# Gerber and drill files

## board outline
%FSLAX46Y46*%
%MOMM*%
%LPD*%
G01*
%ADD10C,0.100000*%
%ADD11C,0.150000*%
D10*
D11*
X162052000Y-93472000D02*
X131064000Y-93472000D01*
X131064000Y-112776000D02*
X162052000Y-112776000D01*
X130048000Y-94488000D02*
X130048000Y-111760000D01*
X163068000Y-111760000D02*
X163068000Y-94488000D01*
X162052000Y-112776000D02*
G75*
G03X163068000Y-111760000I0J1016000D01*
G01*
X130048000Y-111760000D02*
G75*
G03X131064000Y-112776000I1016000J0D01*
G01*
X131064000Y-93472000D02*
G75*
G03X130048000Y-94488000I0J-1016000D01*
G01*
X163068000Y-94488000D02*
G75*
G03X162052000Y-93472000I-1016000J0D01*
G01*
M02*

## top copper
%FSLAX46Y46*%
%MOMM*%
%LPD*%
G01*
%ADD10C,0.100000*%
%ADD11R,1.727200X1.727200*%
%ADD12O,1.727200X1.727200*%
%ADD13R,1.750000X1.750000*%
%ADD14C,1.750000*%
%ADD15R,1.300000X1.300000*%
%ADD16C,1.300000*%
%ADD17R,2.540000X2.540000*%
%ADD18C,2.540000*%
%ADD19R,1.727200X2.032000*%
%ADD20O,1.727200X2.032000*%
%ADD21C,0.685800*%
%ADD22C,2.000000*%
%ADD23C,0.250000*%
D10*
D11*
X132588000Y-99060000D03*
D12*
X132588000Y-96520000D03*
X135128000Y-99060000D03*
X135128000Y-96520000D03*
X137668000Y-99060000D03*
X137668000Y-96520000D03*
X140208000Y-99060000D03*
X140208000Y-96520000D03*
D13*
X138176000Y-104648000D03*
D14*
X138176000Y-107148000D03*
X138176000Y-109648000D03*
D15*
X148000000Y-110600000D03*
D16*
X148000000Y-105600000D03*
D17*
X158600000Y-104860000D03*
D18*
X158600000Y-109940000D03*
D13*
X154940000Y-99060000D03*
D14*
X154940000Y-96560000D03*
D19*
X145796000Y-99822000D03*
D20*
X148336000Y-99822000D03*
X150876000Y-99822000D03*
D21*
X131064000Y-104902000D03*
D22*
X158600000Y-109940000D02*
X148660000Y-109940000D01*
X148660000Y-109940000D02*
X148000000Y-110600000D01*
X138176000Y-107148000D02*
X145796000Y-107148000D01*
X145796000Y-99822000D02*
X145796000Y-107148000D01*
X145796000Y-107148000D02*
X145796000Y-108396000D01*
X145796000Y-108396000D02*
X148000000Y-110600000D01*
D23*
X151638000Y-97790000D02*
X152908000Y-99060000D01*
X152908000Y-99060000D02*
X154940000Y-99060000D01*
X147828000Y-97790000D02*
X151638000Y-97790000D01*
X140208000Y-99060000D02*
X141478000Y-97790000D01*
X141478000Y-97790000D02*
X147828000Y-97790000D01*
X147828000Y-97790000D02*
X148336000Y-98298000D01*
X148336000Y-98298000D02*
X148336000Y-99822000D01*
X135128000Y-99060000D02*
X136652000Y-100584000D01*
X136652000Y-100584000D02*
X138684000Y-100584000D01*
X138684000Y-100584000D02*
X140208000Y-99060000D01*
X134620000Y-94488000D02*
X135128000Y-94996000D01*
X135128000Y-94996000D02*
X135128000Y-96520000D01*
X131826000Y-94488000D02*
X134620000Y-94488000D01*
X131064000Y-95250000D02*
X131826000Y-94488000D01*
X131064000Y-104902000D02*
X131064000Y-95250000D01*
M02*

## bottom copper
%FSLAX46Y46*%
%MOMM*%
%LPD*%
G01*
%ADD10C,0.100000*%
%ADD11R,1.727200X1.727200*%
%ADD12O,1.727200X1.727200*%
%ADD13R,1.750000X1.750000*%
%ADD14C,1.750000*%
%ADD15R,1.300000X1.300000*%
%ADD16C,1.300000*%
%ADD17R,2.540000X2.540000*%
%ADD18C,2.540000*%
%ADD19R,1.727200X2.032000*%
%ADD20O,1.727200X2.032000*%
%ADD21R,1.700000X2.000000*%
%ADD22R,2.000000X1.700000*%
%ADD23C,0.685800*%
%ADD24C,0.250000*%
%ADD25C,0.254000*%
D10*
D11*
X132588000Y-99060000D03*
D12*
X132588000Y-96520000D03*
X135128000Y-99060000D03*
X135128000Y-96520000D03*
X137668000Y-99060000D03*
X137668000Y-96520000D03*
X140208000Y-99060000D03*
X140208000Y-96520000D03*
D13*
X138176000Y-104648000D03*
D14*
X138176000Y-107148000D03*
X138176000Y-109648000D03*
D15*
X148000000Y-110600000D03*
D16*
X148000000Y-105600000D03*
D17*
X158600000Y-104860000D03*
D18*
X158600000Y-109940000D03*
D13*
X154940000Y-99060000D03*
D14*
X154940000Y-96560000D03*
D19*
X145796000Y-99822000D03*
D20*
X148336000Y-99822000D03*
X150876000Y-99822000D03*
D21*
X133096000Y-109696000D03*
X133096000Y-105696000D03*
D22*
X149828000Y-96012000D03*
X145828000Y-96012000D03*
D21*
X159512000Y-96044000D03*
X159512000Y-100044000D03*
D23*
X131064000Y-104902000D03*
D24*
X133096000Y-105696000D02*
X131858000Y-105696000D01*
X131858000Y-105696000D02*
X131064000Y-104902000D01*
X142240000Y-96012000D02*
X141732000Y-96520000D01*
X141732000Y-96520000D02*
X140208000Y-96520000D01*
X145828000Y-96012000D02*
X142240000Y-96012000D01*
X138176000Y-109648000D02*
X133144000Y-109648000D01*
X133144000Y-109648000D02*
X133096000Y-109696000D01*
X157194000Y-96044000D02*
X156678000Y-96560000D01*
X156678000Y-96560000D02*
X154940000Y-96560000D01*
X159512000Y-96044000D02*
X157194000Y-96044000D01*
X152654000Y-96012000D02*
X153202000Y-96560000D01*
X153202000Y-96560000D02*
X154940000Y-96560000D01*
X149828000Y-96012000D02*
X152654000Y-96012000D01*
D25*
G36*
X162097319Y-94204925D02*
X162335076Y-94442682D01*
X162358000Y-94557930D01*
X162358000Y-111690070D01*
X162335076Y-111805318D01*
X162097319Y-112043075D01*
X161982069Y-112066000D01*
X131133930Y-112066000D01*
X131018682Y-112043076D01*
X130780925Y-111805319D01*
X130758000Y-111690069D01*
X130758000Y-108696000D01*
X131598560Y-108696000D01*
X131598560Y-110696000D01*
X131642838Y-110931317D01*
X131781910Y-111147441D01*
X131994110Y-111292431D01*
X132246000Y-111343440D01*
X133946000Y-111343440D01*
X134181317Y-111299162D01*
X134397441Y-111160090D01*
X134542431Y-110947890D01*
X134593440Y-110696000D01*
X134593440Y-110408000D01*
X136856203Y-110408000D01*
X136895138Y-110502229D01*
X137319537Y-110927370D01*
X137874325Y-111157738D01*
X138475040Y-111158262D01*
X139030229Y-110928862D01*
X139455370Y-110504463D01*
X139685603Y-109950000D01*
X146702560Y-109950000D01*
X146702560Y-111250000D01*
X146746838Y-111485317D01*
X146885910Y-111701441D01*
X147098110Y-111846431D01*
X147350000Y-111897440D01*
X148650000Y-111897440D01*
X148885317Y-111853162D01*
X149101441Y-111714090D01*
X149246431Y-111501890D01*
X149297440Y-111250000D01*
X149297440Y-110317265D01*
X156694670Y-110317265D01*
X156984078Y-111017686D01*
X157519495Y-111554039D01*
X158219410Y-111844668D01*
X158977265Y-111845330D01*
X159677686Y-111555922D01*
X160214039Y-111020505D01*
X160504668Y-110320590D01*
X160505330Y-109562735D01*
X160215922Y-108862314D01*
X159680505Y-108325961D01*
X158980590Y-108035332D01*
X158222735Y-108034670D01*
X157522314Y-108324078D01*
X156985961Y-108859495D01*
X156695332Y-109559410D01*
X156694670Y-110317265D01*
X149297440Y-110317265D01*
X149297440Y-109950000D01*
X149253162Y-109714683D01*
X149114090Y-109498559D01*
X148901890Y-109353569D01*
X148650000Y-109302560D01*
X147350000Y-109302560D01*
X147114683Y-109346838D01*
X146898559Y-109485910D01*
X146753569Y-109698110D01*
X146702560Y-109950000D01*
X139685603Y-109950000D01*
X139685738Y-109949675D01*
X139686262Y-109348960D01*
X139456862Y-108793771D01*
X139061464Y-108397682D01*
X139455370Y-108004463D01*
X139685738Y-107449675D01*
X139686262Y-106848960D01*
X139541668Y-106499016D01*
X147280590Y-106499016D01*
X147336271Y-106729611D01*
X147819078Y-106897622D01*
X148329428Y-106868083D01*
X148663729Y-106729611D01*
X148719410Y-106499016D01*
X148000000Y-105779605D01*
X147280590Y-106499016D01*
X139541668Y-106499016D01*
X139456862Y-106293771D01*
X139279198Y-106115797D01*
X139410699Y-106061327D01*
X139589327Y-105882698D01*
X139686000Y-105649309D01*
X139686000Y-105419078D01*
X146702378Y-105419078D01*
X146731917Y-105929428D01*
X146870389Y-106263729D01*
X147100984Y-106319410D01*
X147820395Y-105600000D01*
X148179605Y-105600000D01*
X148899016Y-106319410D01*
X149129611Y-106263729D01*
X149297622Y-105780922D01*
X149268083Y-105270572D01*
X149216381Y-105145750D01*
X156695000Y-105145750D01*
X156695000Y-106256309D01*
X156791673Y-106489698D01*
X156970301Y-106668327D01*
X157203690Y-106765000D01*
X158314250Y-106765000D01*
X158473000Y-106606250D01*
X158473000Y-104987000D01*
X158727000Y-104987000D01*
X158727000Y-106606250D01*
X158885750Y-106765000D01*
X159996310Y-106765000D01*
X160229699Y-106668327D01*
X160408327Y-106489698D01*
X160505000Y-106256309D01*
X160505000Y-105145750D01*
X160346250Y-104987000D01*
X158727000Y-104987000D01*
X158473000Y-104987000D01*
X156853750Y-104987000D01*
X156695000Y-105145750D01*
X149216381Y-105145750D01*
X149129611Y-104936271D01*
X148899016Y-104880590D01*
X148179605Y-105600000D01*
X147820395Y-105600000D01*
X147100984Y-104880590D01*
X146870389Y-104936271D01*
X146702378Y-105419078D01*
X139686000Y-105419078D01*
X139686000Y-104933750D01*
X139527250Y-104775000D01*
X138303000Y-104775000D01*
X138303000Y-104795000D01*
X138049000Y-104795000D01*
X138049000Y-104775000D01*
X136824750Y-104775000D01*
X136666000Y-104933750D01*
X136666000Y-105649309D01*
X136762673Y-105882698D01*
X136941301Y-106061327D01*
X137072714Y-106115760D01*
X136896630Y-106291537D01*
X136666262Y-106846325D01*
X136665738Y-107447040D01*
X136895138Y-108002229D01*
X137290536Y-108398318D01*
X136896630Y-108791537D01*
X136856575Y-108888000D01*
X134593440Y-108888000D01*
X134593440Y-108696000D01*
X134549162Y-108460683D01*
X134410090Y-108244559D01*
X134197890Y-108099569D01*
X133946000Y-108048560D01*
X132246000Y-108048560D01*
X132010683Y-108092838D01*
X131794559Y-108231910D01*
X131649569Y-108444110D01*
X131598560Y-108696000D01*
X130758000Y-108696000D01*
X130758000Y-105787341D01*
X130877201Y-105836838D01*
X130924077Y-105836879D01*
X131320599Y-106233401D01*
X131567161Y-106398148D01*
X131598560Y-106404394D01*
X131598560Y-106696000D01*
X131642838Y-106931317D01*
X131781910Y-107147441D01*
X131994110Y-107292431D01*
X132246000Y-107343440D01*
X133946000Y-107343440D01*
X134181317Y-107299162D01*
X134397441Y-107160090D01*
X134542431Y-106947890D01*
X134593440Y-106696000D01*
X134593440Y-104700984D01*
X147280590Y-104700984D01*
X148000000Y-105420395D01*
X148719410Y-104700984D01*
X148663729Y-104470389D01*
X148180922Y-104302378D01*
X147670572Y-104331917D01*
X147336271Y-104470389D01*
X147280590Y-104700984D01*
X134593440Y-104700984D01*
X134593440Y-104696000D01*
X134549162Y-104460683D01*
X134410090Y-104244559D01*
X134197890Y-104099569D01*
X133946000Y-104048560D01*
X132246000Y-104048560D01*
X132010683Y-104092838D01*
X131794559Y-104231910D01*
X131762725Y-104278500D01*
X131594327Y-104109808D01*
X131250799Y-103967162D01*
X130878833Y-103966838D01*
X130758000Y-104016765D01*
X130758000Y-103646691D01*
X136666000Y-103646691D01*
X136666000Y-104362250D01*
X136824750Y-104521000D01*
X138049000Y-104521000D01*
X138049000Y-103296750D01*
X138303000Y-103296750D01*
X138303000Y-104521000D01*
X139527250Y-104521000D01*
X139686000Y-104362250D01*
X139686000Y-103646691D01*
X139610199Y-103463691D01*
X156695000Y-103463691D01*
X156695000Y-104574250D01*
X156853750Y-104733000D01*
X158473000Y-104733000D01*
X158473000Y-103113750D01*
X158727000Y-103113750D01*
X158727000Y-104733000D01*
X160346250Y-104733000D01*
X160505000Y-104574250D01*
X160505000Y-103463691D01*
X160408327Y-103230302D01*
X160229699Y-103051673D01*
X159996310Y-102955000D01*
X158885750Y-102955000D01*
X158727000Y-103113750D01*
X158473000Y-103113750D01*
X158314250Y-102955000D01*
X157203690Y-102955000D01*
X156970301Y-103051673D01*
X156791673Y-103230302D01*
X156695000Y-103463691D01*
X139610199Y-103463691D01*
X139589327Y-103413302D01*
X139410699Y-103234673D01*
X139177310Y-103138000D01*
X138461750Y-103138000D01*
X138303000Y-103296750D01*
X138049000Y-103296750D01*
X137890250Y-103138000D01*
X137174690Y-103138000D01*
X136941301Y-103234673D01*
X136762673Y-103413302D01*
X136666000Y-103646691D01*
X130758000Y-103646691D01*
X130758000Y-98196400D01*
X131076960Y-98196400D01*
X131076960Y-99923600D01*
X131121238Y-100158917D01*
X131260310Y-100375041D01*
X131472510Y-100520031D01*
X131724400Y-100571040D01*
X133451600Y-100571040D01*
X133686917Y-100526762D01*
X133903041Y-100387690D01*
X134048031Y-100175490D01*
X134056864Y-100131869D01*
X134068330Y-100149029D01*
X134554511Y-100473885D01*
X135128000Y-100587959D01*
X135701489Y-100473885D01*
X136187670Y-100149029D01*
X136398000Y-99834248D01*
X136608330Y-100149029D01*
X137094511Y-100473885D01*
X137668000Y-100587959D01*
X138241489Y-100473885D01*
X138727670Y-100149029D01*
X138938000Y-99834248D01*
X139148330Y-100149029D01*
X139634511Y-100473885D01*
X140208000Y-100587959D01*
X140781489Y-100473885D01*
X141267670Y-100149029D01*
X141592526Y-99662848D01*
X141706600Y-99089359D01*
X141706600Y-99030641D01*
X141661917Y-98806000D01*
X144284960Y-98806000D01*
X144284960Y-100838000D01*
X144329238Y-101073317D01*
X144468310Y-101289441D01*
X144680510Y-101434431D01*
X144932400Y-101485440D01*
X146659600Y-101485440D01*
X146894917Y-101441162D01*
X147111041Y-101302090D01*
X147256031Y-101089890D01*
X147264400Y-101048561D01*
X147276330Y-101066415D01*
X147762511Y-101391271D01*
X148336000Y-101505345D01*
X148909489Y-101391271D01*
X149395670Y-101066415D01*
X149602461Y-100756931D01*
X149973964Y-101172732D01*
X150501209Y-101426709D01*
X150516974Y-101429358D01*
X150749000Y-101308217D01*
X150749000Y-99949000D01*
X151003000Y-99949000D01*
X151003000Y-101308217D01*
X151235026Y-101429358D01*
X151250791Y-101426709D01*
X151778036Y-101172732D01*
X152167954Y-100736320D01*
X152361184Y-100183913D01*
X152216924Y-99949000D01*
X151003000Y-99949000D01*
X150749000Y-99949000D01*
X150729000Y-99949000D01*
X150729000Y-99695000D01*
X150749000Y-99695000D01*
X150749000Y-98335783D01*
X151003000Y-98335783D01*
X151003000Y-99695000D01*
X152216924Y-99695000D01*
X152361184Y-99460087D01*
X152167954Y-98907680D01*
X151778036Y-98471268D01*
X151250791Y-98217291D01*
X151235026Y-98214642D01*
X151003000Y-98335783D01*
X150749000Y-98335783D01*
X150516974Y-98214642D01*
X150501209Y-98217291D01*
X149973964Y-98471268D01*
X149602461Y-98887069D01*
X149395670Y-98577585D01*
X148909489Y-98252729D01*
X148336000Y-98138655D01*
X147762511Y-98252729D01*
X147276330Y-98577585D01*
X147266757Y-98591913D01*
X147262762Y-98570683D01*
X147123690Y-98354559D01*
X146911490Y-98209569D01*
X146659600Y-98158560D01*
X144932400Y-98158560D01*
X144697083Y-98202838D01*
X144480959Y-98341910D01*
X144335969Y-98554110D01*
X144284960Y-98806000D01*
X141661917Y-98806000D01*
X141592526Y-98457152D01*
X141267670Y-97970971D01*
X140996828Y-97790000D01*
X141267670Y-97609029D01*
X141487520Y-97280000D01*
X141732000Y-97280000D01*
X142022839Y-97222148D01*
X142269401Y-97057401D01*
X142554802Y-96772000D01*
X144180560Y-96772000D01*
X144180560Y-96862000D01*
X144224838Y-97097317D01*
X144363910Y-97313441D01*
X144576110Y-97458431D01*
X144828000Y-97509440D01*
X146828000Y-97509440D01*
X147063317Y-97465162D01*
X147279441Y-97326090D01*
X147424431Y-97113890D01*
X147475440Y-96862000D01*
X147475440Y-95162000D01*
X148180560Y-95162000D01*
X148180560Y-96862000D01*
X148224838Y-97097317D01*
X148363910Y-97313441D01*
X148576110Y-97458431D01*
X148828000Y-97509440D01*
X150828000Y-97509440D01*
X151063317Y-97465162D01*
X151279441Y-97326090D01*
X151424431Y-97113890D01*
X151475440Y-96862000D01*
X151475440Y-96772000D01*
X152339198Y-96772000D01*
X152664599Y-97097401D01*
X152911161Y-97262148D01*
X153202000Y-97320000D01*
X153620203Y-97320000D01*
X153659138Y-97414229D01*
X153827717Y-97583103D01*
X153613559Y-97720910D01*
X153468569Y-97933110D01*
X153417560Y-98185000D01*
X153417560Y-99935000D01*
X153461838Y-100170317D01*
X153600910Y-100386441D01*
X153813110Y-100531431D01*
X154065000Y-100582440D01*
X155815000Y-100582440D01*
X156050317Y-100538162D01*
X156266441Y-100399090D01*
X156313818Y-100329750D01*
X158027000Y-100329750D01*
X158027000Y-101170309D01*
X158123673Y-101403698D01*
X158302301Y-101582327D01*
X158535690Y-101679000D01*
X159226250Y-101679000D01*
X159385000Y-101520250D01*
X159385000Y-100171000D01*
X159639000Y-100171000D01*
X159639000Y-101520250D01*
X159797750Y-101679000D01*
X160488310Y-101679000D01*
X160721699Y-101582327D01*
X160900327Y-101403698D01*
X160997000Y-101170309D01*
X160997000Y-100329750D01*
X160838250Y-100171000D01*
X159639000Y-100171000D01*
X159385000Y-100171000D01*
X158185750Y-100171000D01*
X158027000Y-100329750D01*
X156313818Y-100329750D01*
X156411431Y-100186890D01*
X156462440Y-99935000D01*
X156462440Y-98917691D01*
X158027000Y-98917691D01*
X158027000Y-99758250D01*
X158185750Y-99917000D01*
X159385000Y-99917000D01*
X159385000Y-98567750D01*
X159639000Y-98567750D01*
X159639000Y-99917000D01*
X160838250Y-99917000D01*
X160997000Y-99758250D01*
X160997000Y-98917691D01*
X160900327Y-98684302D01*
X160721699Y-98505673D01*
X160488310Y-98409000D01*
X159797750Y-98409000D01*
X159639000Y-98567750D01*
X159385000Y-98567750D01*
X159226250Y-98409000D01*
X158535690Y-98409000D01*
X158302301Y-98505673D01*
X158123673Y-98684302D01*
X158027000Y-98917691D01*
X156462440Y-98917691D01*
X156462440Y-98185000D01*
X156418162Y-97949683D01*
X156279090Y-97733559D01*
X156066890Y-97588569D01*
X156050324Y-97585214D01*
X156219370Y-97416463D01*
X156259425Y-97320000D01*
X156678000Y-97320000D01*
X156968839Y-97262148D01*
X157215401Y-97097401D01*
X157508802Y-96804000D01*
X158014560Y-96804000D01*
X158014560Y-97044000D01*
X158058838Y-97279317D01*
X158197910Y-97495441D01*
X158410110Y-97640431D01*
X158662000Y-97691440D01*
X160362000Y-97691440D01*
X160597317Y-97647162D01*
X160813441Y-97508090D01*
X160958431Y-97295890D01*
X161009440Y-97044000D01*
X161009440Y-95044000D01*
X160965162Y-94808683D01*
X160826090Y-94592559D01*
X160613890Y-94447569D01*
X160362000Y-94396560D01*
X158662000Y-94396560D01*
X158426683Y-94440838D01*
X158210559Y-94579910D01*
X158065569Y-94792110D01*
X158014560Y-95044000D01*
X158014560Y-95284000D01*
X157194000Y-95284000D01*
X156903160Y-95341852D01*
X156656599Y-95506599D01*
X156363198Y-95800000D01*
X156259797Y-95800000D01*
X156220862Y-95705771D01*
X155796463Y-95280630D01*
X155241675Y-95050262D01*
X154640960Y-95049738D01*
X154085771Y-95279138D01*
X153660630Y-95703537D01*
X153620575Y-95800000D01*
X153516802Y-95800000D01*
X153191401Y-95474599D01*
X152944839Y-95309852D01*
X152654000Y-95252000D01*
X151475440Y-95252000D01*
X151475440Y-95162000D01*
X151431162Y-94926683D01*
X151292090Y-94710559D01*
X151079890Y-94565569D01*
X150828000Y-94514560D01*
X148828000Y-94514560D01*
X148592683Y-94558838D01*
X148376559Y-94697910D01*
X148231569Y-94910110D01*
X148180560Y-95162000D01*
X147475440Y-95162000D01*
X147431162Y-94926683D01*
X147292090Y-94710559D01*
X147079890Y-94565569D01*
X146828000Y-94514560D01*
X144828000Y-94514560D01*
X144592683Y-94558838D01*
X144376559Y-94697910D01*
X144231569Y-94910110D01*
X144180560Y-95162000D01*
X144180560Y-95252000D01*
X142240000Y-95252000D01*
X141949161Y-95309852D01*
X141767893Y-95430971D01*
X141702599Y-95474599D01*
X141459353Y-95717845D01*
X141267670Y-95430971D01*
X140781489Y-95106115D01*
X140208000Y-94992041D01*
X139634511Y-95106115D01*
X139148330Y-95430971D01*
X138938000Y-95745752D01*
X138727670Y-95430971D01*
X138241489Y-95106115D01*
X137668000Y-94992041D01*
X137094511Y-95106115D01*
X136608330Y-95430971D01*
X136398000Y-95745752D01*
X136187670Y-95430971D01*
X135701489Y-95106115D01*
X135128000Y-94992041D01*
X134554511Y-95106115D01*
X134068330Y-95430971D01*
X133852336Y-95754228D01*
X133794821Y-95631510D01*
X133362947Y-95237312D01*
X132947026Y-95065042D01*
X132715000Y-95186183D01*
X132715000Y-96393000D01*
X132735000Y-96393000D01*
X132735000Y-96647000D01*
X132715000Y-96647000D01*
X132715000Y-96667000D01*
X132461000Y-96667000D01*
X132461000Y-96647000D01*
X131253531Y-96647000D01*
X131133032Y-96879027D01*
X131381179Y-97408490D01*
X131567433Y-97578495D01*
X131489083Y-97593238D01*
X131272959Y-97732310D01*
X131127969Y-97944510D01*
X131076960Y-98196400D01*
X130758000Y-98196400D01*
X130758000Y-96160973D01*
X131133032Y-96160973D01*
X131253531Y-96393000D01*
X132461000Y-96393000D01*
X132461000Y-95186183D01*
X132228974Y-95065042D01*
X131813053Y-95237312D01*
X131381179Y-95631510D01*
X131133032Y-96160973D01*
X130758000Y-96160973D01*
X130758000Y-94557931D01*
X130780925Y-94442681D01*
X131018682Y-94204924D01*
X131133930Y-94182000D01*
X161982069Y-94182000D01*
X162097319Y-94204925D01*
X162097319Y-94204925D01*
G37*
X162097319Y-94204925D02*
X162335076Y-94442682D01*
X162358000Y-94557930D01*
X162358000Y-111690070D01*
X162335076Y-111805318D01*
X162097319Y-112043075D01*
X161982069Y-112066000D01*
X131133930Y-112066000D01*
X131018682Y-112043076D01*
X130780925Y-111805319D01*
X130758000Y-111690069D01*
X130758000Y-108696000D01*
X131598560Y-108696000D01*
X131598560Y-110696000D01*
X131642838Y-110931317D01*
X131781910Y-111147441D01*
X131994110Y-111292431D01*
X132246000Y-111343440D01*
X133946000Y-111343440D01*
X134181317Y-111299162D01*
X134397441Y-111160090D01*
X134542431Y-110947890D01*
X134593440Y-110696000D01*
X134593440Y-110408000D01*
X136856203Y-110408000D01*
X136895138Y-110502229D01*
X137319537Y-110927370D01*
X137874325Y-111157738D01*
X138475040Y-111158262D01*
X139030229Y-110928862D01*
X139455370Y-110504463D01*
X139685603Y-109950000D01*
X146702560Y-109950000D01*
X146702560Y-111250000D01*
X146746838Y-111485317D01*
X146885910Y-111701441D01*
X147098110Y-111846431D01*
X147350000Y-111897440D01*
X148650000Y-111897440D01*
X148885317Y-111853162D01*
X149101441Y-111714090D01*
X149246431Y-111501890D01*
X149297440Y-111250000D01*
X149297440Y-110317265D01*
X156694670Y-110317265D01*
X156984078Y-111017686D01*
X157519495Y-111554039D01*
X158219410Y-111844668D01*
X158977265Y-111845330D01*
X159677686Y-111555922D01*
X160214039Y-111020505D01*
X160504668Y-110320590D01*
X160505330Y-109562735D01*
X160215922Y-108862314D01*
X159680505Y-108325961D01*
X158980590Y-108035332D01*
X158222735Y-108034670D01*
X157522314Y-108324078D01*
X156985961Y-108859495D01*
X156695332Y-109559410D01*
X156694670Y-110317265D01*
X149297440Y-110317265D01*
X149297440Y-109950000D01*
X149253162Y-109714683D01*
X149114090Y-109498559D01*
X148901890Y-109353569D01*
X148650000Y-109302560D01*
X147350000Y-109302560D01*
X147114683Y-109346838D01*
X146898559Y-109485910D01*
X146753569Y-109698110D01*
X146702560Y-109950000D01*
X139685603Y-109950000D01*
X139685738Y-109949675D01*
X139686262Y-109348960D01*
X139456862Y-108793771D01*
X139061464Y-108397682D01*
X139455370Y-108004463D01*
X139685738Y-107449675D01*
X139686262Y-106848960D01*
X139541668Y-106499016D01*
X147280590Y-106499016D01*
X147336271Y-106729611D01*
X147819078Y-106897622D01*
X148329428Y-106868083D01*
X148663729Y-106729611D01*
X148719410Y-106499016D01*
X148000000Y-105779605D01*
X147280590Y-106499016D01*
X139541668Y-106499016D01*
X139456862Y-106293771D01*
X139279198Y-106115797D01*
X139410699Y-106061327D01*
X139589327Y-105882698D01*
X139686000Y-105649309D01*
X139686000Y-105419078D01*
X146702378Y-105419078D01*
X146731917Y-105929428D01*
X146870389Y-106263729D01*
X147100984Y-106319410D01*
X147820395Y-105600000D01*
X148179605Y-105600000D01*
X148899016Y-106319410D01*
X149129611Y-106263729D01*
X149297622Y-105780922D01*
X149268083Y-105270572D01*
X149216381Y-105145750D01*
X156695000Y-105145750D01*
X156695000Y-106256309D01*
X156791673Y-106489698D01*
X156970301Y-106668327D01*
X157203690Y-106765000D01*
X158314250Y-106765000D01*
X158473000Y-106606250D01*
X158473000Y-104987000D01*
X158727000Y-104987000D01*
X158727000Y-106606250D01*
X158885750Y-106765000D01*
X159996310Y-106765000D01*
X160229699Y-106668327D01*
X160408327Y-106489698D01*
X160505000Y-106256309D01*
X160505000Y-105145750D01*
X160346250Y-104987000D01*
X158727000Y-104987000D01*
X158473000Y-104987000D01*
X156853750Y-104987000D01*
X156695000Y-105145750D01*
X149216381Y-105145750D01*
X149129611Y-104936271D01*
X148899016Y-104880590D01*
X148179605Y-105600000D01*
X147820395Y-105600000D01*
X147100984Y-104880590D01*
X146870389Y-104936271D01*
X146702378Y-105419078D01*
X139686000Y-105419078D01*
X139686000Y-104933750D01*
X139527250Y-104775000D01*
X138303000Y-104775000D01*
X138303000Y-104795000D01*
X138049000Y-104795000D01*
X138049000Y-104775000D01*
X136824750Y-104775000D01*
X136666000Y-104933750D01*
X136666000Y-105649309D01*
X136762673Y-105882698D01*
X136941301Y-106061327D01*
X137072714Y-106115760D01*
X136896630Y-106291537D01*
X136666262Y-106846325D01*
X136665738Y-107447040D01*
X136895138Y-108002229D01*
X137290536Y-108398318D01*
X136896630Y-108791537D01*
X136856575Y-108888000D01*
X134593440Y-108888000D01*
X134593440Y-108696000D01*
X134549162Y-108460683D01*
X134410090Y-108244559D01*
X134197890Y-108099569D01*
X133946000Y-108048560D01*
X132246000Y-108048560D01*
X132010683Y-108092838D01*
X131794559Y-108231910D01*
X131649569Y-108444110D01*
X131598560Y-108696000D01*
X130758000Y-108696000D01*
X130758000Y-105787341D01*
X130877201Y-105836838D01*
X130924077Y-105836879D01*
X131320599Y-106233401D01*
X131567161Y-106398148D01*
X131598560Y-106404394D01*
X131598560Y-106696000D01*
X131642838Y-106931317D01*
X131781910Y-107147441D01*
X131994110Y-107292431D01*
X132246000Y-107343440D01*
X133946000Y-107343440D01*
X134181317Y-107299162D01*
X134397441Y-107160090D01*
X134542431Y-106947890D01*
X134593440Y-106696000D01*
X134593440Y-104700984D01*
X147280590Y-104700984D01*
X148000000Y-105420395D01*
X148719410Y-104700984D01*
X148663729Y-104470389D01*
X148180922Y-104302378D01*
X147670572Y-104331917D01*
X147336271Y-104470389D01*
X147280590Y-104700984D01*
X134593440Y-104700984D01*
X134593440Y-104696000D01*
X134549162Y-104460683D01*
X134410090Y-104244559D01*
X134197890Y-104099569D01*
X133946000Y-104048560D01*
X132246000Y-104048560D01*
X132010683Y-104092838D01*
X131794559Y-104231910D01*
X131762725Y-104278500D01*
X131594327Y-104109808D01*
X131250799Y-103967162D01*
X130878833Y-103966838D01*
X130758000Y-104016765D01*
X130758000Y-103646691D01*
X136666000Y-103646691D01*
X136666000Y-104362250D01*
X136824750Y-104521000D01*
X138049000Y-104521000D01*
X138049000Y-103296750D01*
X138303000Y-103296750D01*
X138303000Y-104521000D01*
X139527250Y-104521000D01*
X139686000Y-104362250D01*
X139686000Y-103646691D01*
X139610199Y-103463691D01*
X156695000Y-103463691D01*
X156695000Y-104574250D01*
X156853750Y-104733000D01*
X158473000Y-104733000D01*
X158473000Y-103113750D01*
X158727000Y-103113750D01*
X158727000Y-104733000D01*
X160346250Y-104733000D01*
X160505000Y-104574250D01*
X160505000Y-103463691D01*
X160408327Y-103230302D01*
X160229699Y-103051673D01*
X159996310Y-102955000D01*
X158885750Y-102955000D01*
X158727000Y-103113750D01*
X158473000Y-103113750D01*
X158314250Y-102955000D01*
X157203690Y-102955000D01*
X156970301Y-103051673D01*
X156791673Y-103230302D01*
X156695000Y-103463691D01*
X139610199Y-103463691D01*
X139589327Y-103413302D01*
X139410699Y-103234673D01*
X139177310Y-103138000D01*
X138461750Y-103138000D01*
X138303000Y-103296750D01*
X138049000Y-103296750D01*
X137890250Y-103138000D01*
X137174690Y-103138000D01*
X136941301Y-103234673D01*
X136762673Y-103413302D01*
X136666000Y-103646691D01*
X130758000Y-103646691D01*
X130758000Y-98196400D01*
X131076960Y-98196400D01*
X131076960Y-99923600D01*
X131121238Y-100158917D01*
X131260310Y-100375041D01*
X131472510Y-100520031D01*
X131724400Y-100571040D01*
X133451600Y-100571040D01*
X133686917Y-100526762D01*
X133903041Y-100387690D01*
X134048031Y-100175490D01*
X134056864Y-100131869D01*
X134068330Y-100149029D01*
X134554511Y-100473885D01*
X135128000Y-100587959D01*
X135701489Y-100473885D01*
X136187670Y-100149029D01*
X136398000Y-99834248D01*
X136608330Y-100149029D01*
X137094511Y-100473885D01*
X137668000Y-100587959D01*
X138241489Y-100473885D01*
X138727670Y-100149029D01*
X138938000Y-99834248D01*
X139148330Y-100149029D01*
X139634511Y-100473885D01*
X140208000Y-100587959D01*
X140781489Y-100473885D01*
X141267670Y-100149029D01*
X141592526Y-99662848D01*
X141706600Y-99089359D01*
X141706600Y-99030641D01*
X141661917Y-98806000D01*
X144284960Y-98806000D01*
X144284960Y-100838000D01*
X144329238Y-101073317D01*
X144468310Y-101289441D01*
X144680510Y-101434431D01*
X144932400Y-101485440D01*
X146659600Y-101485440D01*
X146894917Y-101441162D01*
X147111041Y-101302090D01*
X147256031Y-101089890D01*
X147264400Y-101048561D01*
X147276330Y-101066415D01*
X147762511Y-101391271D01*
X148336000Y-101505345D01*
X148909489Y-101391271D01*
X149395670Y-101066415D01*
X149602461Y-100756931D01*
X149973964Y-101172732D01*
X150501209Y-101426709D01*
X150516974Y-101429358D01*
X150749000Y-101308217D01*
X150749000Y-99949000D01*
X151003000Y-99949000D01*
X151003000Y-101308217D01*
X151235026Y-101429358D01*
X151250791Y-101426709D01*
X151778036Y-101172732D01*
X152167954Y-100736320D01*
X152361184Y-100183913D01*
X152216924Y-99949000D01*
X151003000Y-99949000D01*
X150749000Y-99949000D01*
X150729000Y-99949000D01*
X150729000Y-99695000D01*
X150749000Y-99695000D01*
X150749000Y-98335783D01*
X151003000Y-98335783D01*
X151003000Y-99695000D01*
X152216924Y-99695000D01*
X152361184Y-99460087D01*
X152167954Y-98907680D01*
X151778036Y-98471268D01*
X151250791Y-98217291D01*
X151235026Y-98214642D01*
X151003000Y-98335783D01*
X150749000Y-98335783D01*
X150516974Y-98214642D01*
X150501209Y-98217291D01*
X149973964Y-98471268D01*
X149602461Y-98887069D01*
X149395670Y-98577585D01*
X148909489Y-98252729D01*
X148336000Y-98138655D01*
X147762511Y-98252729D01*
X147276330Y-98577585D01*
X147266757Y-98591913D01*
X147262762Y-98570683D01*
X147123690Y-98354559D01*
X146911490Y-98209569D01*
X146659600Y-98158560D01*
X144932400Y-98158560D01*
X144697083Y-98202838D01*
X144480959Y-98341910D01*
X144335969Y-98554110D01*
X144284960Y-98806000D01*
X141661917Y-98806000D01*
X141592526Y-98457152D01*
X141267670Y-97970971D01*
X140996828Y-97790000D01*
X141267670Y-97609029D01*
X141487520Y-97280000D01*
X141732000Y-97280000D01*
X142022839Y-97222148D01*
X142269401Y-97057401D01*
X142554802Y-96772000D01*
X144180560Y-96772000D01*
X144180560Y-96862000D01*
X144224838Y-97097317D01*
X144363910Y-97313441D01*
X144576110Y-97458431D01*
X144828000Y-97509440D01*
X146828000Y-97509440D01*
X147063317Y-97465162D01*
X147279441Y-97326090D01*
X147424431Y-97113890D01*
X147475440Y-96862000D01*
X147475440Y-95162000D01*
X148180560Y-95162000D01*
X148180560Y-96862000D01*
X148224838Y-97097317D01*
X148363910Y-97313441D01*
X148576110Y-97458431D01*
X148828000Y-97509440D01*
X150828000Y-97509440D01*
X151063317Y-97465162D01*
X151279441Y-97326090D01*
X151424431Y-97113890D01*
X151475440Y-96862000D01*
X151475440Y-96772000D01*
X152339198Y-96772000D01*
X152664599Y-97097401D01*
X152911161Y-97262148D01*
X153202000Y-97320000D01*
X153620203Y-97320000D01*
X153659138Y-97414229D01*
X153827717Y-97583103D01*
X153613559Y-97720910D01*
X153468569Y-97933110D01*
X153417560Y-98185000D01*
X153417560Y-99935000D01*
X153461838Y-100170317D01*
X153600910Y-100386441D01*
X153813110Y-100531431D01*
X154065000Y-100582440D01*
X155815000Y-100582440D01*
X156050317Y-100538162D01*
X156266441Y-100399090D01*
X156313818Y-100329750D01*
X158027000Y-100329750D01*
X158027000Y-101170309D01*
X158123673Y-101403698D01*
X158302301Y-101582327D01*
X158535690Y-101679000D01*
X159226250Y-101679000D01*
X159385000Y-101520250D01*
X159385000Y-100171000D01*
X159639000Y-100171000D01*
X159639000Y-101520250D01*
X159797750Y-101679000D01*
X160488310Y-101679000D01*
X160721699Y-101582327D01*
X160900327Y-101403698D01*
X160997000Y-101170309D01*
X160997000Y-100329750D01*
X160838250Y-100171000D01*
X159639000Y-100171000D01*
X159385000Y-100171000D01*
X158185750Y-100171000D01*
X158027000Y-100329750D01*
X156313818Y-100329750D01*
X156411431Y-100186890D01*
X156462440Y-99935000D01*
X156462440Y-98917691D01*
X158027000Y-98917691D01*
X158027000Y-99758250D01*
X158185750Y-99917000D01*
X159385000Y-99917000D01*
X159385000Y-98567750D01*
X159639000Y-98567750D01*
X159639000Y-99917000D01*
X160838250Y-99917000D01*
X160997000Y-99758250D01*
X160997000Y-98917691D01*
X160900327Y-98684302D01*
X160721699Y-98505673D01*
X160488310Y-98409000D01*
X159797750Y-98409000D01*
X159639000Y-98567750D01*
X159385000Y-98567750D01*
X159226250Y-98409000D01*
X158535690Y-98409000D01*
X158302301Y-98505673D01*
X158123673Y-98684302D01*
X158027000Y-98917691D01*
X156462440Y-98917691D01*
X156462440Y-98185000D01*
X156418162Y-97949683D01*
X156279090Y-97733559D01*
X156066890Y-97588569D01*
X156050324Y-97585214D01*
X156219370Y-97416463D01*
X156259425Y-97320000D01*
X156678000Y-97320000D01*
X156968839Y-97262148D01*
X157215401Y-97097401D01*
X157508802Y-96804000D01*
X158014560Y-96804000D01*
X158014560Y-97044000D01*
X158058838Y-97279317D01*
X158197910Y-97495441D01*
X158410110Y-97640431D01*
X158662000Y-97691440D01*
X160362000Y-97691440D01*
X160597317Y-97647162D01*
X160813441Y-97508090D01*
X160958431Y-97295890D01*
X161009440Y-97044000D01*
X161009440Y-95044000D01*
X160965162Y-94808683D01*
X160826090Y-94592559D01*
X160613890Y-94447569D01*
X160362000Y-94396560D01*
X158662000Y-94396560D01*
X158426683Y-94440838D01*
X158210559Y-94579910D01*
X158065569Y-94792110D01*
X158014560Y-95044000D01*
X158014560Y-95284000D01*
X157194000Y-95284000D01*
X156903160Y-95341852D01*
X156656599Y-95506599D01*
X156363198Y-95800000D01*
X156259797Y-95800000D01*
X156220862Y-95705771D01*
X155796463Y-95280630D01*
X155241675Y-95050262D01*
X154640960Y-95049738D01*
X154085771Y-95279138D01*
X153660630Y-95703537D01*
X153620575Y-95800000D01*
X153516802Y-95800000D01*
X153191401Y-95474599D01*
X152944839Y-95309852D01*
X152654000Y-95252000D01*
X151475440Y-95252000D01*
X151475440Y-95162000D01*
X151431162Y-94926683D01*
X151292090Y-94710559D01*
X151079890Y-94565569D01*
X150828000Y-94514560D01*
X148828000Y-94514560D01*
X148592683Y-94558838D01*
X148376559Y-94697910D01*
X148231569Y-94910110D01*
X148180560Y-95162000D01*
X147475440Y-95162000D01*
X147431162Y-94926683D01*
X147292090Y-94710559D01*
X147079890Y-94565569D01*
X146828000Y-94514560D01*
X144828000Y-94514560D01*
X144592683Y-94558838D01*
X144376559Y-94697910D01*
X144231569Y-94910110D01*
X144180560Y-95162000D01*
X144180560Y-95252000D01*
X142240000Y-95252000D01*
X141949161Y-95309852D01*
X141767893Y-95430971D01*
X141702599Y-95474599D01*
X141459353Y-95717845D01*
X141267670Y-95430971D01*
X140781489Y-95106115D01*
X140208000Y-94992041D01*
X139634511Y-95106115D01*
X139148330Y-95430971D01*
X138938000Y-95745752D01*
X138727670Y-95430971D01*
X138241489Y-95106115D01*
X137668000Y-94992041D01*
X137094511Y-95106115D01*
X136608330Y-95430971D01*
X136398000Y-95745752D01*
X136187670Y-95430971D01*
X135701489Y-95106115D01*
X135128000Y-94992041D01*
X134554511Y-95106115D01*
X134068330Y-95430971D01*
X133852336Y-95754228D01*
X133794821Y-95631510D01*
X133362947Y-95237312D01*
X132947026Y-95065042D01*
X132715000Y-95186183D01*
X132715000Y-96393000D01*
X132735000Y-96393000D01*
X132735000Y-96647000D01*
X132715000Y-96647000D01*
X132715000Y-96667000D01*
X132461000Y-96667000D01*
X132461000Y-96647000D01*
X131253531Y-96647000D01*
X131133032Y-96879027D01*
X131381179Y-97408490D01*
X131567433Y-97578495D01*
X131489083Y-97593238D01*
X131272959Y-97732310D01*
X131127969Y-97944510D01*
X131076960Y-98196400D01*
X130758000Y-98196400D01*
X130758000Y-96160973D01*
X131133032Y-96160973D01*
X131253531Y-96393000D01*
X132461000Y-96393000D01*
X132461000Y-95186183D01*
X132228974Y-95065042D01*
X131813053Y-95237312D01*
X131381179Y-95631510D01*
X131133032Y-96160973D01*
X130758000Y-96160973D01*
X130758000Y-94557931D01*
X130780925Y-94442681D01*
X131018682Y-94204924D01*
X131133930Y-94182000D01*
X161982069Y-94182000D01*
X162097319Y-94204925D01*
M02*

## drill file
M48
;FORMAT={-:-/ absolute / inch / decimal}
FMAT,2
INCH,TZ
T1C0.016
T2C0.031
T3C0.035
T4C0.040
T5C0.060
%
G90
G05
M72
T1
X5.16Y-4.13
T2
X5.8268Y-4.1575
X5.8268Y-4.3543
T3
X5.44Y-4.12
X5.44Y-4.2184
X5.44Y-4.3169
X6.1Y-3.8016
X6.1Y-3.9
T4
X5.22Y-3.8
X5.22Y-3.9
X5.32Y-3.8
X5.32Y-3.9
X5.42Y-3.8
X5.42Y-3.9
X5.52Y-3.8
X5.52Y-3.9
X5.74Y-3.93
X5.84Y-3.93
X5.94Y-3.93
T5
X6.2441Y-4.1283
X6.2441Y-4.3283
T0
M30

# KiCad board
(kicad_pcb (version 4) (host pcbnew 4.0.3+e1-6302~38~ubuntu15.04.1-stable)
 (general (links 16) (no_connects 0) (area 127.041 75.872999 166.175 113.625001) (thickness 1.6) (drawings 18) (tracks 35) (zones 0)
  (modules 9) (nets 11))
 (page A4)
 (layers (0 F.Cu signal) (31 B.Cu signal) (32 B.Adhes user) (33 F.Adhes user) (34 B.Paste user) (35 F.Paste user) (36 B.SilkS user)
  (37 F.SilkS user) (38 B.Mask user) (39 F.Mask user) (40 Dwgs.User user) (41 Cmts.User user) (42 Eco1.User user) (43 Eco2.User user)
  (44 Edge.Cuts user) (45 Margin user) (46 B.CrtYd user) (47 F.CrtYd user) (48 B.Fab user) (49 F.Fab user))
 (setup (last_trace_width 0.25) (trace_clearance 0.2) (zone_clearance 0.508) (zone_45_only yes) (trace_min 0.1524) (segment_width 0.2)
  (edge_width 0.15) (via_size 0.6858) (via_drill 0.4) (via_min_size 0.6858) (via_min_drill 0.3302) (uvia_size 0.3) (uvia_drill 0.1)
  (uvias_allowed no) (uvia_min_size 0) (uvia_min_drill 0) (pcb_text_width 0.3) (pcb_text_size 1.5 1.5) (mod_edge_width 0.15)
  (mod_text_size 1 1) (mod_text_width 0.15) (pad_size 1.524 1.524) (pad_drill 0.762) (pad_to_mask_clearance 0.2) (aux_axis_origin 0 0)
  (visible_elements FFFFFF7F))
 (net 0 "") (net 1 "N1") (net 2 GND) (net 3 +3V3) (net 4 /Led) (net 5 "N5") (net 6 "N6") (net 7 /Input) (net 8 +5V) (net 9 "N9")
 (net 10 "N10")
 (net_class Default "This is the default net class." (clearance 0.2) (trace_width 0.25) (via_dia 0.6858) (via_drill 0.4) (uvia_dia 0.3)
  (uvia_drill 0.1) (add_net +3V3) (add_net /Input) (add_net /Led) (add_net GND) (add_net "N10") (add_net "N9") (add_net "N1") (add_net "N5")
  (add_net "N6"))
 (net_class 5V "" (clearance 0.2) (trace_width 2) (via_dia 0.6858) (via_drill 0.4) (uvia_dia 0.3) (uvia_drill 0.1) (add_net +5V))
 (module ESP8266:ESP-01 (layer F.Cu) (at 132.588 99.06 90)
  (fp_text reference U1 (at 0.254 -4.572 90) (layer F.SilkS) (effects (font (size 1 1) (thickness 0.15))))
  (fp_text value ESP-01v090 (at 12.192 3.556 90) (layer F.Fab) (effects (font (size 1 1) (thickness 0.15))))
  (pad 1 thru_hole rect (at 0 0 90) (size 1.7272 1.7272) (drill 1.016) (layers *.Cu *.Mask F.SilkS) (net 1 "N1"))
  (pad 2 thru_hole oval (at 2.54 0 90) (size 1.7272 1.7272) (drill 1.016) (layers *.Cu *.Mask F.SilkS) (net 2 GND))
  (pad 3 thru_hole oval (at 0 2.54 90) (size 1.7272 1.7272) (drill 1.016) (layers *.Cu *.Mask F.SilkS) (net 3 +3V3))
  (pad 4 thru_hole oval (at 2.54 2.54 90) (size 1.7272 1.7272) (drill 1.016) (layers *.Cu *.Mask F.SilkS) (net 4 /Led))
  (pad 5 thru_hole oval (at 0 5.08 90) (size 1.7272 1.7272) (drill 1.016) (layers *.Cu *.Mask F.SilkS) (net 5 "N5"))
  (pad 6 thru_hole oval (at 2.54 5.08 90) (size 1.7272 1.7272) (drill 1.016) (layers *.Cu *.Mask F.SilkS) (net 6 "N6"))
  (pad 7 thru_hole oval (at 0 7.62 90) (size 1.7272 1.7272) (drill 1.016) (layers *.Cu *.Mask F.SilkS) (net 3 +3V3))
  (pad 8 thru_hole oval (at 2.54 7.62 90) (size 1.7272 1.7272) (drill 1.016) (layers *.Cu *.Mask F.SilkS) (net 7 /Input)))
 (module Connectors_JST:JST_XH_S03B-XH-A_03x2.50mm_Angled (layer F.Cu) (at 138.176 104.648 270)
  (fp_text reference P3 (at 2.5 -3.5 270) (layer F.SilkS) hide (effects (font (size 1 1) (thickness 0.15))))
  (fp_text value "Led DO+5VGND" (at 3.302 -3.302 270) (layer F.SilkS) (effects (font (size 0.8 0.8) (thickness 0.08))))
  (pad 1 thru_hole rect (at 0 0 270) (size 1.75 1.75) (drill 0.9) (layers *.Cu *.Mask F.SilkS) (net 2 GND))
  (pad 2 thru_hole circle (at 2.5 0 270) (size 1.75 1.75) (drill 0.9) (layers *.Cu *.Mask F.SilkS) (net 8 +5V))
  (pad 3 thru_hole circle (at 5 0 270) (size 1.75 1.75) (drill 0.9) (layers *.Cu *.Mask F.SilkS) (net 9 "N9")))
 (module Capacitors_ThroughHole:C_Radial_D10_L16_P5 (layer F.Cu) (at 148 110.6 90)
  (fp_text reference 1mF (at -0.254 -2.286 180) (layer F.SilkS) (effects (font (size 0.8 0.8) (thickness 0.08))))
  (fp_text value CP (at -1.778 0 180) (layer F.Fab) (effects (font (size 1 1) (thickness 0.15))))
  (pad 1 thru_hole rect (at 0 0 90) (size 1.3 1.3) (drill 0.8) (layers *.Cu *.Mask F.SilkS) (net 8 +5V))
  (pad 2 thru_hole circle (at 5 0 90) (size 1.3 1.3) (drill 0.8) (layers *.Cu *.Mask F.SilkS) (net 2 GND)))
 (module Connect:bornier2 (layer F.Cu) (at 158.6 107.4 270)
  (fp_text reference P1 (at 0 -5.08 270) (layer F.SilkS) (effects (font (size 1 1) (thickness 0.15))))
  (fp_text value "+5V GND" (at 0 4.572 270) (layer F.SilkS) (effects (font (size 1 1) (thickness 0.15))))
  (pad 1 thru_hole rect (at -2.54 0 270) (size 2.54 2.54) (drill 1.524) (layers *.Cu *.Mask F.SilkS) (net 2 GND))
  (pad 2 thru_hole circle (at 2.54 0 270) (size 2.54 2.54) (drill 1.524) (layers *.Cu *.Mask F.SilkS) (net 8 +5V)))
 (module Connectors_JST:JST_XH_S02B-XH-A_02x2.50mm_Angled (layer F.Cu) (at 154.94 99.06 90)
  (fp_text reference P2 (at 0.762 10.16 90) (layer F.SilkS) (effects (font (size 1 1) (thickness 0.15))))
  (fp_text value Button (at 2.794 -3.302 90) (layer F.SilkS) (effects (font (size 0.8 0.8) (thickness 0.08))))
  (pad 1 thru_hole rect (at 0 0 90) (size 1.75 1.75) (drill 0.9) (layers *.Cu *.Mask F.SilkS) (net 3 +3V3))
  (pad 2 thru_hole circle (at 2.5 0 90) (size 1.75 1.75) (drill 0.9) (layers *.Cu *.Mask F.SilkS) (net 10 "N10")))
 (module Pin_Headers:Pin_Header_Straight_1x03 (layer F.Cu) (at 145.796 99.822 90)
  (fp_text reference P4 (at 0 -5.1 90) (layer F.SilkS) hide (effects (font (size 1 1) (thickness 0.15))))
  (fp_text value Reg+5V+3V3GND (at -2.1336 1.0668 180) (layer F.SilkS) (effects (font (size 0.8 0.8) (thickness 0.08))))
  (pad 1 thru_hole rect (at 0 0 90) (size 2.032 1.7272) (drill 1.016) (layers *.Cu *.Mask F.SilkS) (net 8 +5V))
  (pad 2 thru_hole oval (at 0 2.54 90) (size 2.032 1.7272) (drill 1.016) (layers *.Cu *.Mask F.SilkS) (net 3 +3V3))
  (pad 3 thru_hole oval (at 0 5.08 90) (size 2.032 1.7272) (drill 1.016) (layers *.Cu *.Mask F.SilkS) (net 2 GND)))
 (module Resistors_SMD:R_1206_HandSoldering (layer B.Cu) (at 133.096 107.696 90)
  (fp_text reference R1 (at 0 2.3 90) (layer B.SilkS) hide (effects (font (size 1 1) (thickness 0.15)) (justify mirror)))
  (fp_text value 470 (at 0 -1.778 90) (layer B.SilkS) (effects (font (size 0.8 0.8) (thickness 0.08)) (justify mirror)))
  (pad 1 smd rect (at -2 0 90) (size 2 1.7) (layers B.Cu B.Paste B.Mask) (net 9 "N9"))
  (pad 2 smd rect (at 2 0 90) (size 2 1.7) (layers B.Cu B.Paste B.Mask) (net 4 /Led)))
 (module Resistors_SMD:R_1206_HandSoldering (layer B.Cu) (at 147.828 96.012 180)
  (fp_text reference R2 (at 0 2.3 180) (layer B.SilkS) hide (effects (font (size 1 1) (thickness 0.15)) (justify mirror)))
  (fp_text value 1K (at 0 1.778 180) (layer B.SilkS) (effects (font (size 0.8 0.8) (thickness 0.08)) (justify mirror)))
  (pad 1 smd rect (at -2 0 180) (size 2 1.7) (layers B.Cu B.Paste B.Mask) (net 10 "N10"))
  (pad 2 smd rect (at 2 0 180) (size 2 1.7) (layers B.Cu B.Paste B.Mask) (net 7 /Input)))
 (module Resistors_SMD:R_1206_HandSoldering (layer B.Cu) (at 159.512 98.044 270)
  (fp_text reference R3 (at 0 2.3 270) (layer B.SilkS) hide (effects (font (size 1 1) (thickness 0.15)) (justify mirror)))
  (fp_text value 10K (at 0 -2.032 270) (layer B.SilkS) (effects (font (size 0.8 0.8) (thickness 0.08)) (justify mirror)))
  (pad 1 smd rect (at -2 0 270) (size 2 1.7) (layers B.Cu B.Paste B.Mask) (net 10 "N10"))
  (pad 2 smd rect (at 2 0 270) (size 2 1.7) (layers B.Cu B.Paste B.Mask) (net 2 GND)))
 (gr_line (start 162.052 93.472) (end 131.064 93.472) (angle 90) (layer Edge.Cuts) (width 0.15))
 (gr_line (start 131.064 112.776) (end 162.052 112.776) (angle 90) (layer Edge.Cuts) (width 0.15))
 (gr_line (start 130.048 94.488) (end 130.048 111.76) (angle 90) (layer Edge.Cuts) (width 0.15))
 (gr_line (start 163.068 111.76) (end 163.068 94.488) (angle 90) (layer Edge.Cuts) (width 0.15))
 (gr_arc (start 162.052 111.76) (end 163.068 111.76) (angle 90) (layer Edge.Cuts) (width 0.15))
 (gr_arc (start 131.064 111.76) (end 131.064 112.776) (angle 90) (layer Edge.Cuts) (width 0.15))
 (gr_arc (start 131.064 94.488) (end 130.048 94.488) (angle 90) (layer Edge.Cuts) (width 0.15))
 (gr_arc (start 162.052 94.488) (end 162.052 93.472) (angle 90) (layer Edge.Cuts) (width 0.15))
 (segment (start 158.6 109.94) (end 148.66 109.94) (width 2) (layer F.Cu) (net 8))
 (segment (start 148.66 109.94) (end 148 110.6) (width 2) (layer F.Cu) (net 8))
 (segment (start 138.176 107.148) (end 145.796 107.148) (width 2) (layer F.Cu) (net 8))
 (segment (start 145.796 99.822) (end 145.796 107.148) (width 2) (layer F.Cu) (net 8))
 (segment (start 145.796 107.148) (end 145.796 108.396) (width 2) (layer F.Cu) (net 8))
 (segment (start 145.796 108.396) (end 148 110.6) (width 2) (layer F.Cu) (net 8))
 (segment (start 151.638 97.79) (end 152.908 99.06) (width 0.25) (layer F.Cu) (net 3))
 (segment (start 152.908 99.06) (end 154.94 99.06) (width 0.25) (layer F.Cu) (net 3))
 (segment (start 147.828 97.79) (end 151.638 97.79) (width 0.25) (layer F.Cu) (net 3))
 (segment (start 140.208 99.06) (end 141.478 97.79) (width 0.25) (layer F.Cu) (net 3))
 (segment (start 141.478 97.79) (end 147.828 97.79) (width 0.25) (layer F.Cu) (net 3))
 (segment (start 147.828 97.79) (end 148.336 98.298) (width 0.25) (layer F.Cu) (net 3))
 (segment (start 148.336 98.298) (end 148.336 99.822) (width 0.25) (layer F.Cu) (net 3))
 (segment (start 135.128 99.06) (end 136.652 100.584) (width 0.25) (layer F.Cu) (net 3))
 (segment (start 136.652 100.584) (end 138.684 100.584) (width 0.25) (layer F.Cu) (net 3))
 (segment (start 138.684 100.584) (end 140.208 99.06) (width 0.25) (layer F.Cu) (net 3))
 (segment (start 134.62 94.488) (end 135.128 94.996) (width 0.25) (layer F.Cu) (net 4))
 (segment (start 135.128 94.996) (end 135.128 96.52) (width 0.25) (layer F.Cu) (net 4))
 (segment (start 131.826 94.488) (end 134.62 94.488) (width 0.25) (layer F.Cu) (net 4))
 (segment (start 131.064 95.25) (end 131.826 94.488) (width 0.25) (layer F.Cu) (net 4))
 (segment (start 131.064 104.902) (end 131.064 95.25) (width 0.25) (layer F.Cu) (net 4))
 (segment (start 133.096 105.696) (end 131.858 105.696) (width 0.25) (layer B.Cu) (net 4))
 (segment (start 131.858 105.696) (end 131.064 104.902) (width 0.25) (layer B.Cu) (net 4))
 (via (at 131.064 104.902) (size 0.6858) (drill 0.4) (layers F.Cu B.Cu) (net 4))
 (segment (start 142.24 96.012) (end 141.732 96.52) (width 0.25) (layer B.Cu) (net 7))
 (segment (start 141.732 96.52) (end 140.208 96.52) (width 0.25) (layer B.Cu) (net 7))
 (segment (start 145.828 96.012) (end 142.24 96.012) (width 0.25) (layer B.Cu) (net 7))
 (segment (start 138.176 109.648) (end 133.144 109.648) (width 0.25) (layer B.Cu) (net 9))
 (segment (start 133.144 109.648) (end 133.096 109.696) (width 0.25) (layer B.Cu) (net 9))
 (segment (start 157.194 96.044) (end 156.678 96.56) (width 0.25) (layer B.Cu) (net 10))
 (segment (start 156.678 96.56) (end 154.94 96.56) (width 0.25) (layer B.Cu) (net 10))
 (segment (start 159.512 96.044) (end 157.194 96.044) (width 0.25) (layer B.Cu) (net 10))
 (segment (start 152.654 96.012) (end 153.202 96.56) (width 0.25) (layer B.Cu) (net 10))
 (segment (start 153.202 96.56) (end 154.94 96.56) (width 0.25) (layer B.Cu) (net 10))
 (segment (start 149.828 96.012) (end 152.654 96.012) (width 0.25) (layer B.Cu) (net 10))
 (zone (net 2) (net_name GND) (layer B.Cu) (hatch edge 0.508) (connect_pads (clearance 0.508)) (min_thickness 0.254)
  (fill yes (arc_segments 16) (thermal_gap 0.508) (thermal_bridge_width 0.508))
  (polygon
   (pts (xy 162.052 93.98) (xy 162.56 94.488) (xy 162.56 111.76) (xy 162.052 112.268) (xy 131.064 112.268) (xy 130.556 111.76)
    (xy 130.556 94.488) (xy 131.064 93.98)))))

